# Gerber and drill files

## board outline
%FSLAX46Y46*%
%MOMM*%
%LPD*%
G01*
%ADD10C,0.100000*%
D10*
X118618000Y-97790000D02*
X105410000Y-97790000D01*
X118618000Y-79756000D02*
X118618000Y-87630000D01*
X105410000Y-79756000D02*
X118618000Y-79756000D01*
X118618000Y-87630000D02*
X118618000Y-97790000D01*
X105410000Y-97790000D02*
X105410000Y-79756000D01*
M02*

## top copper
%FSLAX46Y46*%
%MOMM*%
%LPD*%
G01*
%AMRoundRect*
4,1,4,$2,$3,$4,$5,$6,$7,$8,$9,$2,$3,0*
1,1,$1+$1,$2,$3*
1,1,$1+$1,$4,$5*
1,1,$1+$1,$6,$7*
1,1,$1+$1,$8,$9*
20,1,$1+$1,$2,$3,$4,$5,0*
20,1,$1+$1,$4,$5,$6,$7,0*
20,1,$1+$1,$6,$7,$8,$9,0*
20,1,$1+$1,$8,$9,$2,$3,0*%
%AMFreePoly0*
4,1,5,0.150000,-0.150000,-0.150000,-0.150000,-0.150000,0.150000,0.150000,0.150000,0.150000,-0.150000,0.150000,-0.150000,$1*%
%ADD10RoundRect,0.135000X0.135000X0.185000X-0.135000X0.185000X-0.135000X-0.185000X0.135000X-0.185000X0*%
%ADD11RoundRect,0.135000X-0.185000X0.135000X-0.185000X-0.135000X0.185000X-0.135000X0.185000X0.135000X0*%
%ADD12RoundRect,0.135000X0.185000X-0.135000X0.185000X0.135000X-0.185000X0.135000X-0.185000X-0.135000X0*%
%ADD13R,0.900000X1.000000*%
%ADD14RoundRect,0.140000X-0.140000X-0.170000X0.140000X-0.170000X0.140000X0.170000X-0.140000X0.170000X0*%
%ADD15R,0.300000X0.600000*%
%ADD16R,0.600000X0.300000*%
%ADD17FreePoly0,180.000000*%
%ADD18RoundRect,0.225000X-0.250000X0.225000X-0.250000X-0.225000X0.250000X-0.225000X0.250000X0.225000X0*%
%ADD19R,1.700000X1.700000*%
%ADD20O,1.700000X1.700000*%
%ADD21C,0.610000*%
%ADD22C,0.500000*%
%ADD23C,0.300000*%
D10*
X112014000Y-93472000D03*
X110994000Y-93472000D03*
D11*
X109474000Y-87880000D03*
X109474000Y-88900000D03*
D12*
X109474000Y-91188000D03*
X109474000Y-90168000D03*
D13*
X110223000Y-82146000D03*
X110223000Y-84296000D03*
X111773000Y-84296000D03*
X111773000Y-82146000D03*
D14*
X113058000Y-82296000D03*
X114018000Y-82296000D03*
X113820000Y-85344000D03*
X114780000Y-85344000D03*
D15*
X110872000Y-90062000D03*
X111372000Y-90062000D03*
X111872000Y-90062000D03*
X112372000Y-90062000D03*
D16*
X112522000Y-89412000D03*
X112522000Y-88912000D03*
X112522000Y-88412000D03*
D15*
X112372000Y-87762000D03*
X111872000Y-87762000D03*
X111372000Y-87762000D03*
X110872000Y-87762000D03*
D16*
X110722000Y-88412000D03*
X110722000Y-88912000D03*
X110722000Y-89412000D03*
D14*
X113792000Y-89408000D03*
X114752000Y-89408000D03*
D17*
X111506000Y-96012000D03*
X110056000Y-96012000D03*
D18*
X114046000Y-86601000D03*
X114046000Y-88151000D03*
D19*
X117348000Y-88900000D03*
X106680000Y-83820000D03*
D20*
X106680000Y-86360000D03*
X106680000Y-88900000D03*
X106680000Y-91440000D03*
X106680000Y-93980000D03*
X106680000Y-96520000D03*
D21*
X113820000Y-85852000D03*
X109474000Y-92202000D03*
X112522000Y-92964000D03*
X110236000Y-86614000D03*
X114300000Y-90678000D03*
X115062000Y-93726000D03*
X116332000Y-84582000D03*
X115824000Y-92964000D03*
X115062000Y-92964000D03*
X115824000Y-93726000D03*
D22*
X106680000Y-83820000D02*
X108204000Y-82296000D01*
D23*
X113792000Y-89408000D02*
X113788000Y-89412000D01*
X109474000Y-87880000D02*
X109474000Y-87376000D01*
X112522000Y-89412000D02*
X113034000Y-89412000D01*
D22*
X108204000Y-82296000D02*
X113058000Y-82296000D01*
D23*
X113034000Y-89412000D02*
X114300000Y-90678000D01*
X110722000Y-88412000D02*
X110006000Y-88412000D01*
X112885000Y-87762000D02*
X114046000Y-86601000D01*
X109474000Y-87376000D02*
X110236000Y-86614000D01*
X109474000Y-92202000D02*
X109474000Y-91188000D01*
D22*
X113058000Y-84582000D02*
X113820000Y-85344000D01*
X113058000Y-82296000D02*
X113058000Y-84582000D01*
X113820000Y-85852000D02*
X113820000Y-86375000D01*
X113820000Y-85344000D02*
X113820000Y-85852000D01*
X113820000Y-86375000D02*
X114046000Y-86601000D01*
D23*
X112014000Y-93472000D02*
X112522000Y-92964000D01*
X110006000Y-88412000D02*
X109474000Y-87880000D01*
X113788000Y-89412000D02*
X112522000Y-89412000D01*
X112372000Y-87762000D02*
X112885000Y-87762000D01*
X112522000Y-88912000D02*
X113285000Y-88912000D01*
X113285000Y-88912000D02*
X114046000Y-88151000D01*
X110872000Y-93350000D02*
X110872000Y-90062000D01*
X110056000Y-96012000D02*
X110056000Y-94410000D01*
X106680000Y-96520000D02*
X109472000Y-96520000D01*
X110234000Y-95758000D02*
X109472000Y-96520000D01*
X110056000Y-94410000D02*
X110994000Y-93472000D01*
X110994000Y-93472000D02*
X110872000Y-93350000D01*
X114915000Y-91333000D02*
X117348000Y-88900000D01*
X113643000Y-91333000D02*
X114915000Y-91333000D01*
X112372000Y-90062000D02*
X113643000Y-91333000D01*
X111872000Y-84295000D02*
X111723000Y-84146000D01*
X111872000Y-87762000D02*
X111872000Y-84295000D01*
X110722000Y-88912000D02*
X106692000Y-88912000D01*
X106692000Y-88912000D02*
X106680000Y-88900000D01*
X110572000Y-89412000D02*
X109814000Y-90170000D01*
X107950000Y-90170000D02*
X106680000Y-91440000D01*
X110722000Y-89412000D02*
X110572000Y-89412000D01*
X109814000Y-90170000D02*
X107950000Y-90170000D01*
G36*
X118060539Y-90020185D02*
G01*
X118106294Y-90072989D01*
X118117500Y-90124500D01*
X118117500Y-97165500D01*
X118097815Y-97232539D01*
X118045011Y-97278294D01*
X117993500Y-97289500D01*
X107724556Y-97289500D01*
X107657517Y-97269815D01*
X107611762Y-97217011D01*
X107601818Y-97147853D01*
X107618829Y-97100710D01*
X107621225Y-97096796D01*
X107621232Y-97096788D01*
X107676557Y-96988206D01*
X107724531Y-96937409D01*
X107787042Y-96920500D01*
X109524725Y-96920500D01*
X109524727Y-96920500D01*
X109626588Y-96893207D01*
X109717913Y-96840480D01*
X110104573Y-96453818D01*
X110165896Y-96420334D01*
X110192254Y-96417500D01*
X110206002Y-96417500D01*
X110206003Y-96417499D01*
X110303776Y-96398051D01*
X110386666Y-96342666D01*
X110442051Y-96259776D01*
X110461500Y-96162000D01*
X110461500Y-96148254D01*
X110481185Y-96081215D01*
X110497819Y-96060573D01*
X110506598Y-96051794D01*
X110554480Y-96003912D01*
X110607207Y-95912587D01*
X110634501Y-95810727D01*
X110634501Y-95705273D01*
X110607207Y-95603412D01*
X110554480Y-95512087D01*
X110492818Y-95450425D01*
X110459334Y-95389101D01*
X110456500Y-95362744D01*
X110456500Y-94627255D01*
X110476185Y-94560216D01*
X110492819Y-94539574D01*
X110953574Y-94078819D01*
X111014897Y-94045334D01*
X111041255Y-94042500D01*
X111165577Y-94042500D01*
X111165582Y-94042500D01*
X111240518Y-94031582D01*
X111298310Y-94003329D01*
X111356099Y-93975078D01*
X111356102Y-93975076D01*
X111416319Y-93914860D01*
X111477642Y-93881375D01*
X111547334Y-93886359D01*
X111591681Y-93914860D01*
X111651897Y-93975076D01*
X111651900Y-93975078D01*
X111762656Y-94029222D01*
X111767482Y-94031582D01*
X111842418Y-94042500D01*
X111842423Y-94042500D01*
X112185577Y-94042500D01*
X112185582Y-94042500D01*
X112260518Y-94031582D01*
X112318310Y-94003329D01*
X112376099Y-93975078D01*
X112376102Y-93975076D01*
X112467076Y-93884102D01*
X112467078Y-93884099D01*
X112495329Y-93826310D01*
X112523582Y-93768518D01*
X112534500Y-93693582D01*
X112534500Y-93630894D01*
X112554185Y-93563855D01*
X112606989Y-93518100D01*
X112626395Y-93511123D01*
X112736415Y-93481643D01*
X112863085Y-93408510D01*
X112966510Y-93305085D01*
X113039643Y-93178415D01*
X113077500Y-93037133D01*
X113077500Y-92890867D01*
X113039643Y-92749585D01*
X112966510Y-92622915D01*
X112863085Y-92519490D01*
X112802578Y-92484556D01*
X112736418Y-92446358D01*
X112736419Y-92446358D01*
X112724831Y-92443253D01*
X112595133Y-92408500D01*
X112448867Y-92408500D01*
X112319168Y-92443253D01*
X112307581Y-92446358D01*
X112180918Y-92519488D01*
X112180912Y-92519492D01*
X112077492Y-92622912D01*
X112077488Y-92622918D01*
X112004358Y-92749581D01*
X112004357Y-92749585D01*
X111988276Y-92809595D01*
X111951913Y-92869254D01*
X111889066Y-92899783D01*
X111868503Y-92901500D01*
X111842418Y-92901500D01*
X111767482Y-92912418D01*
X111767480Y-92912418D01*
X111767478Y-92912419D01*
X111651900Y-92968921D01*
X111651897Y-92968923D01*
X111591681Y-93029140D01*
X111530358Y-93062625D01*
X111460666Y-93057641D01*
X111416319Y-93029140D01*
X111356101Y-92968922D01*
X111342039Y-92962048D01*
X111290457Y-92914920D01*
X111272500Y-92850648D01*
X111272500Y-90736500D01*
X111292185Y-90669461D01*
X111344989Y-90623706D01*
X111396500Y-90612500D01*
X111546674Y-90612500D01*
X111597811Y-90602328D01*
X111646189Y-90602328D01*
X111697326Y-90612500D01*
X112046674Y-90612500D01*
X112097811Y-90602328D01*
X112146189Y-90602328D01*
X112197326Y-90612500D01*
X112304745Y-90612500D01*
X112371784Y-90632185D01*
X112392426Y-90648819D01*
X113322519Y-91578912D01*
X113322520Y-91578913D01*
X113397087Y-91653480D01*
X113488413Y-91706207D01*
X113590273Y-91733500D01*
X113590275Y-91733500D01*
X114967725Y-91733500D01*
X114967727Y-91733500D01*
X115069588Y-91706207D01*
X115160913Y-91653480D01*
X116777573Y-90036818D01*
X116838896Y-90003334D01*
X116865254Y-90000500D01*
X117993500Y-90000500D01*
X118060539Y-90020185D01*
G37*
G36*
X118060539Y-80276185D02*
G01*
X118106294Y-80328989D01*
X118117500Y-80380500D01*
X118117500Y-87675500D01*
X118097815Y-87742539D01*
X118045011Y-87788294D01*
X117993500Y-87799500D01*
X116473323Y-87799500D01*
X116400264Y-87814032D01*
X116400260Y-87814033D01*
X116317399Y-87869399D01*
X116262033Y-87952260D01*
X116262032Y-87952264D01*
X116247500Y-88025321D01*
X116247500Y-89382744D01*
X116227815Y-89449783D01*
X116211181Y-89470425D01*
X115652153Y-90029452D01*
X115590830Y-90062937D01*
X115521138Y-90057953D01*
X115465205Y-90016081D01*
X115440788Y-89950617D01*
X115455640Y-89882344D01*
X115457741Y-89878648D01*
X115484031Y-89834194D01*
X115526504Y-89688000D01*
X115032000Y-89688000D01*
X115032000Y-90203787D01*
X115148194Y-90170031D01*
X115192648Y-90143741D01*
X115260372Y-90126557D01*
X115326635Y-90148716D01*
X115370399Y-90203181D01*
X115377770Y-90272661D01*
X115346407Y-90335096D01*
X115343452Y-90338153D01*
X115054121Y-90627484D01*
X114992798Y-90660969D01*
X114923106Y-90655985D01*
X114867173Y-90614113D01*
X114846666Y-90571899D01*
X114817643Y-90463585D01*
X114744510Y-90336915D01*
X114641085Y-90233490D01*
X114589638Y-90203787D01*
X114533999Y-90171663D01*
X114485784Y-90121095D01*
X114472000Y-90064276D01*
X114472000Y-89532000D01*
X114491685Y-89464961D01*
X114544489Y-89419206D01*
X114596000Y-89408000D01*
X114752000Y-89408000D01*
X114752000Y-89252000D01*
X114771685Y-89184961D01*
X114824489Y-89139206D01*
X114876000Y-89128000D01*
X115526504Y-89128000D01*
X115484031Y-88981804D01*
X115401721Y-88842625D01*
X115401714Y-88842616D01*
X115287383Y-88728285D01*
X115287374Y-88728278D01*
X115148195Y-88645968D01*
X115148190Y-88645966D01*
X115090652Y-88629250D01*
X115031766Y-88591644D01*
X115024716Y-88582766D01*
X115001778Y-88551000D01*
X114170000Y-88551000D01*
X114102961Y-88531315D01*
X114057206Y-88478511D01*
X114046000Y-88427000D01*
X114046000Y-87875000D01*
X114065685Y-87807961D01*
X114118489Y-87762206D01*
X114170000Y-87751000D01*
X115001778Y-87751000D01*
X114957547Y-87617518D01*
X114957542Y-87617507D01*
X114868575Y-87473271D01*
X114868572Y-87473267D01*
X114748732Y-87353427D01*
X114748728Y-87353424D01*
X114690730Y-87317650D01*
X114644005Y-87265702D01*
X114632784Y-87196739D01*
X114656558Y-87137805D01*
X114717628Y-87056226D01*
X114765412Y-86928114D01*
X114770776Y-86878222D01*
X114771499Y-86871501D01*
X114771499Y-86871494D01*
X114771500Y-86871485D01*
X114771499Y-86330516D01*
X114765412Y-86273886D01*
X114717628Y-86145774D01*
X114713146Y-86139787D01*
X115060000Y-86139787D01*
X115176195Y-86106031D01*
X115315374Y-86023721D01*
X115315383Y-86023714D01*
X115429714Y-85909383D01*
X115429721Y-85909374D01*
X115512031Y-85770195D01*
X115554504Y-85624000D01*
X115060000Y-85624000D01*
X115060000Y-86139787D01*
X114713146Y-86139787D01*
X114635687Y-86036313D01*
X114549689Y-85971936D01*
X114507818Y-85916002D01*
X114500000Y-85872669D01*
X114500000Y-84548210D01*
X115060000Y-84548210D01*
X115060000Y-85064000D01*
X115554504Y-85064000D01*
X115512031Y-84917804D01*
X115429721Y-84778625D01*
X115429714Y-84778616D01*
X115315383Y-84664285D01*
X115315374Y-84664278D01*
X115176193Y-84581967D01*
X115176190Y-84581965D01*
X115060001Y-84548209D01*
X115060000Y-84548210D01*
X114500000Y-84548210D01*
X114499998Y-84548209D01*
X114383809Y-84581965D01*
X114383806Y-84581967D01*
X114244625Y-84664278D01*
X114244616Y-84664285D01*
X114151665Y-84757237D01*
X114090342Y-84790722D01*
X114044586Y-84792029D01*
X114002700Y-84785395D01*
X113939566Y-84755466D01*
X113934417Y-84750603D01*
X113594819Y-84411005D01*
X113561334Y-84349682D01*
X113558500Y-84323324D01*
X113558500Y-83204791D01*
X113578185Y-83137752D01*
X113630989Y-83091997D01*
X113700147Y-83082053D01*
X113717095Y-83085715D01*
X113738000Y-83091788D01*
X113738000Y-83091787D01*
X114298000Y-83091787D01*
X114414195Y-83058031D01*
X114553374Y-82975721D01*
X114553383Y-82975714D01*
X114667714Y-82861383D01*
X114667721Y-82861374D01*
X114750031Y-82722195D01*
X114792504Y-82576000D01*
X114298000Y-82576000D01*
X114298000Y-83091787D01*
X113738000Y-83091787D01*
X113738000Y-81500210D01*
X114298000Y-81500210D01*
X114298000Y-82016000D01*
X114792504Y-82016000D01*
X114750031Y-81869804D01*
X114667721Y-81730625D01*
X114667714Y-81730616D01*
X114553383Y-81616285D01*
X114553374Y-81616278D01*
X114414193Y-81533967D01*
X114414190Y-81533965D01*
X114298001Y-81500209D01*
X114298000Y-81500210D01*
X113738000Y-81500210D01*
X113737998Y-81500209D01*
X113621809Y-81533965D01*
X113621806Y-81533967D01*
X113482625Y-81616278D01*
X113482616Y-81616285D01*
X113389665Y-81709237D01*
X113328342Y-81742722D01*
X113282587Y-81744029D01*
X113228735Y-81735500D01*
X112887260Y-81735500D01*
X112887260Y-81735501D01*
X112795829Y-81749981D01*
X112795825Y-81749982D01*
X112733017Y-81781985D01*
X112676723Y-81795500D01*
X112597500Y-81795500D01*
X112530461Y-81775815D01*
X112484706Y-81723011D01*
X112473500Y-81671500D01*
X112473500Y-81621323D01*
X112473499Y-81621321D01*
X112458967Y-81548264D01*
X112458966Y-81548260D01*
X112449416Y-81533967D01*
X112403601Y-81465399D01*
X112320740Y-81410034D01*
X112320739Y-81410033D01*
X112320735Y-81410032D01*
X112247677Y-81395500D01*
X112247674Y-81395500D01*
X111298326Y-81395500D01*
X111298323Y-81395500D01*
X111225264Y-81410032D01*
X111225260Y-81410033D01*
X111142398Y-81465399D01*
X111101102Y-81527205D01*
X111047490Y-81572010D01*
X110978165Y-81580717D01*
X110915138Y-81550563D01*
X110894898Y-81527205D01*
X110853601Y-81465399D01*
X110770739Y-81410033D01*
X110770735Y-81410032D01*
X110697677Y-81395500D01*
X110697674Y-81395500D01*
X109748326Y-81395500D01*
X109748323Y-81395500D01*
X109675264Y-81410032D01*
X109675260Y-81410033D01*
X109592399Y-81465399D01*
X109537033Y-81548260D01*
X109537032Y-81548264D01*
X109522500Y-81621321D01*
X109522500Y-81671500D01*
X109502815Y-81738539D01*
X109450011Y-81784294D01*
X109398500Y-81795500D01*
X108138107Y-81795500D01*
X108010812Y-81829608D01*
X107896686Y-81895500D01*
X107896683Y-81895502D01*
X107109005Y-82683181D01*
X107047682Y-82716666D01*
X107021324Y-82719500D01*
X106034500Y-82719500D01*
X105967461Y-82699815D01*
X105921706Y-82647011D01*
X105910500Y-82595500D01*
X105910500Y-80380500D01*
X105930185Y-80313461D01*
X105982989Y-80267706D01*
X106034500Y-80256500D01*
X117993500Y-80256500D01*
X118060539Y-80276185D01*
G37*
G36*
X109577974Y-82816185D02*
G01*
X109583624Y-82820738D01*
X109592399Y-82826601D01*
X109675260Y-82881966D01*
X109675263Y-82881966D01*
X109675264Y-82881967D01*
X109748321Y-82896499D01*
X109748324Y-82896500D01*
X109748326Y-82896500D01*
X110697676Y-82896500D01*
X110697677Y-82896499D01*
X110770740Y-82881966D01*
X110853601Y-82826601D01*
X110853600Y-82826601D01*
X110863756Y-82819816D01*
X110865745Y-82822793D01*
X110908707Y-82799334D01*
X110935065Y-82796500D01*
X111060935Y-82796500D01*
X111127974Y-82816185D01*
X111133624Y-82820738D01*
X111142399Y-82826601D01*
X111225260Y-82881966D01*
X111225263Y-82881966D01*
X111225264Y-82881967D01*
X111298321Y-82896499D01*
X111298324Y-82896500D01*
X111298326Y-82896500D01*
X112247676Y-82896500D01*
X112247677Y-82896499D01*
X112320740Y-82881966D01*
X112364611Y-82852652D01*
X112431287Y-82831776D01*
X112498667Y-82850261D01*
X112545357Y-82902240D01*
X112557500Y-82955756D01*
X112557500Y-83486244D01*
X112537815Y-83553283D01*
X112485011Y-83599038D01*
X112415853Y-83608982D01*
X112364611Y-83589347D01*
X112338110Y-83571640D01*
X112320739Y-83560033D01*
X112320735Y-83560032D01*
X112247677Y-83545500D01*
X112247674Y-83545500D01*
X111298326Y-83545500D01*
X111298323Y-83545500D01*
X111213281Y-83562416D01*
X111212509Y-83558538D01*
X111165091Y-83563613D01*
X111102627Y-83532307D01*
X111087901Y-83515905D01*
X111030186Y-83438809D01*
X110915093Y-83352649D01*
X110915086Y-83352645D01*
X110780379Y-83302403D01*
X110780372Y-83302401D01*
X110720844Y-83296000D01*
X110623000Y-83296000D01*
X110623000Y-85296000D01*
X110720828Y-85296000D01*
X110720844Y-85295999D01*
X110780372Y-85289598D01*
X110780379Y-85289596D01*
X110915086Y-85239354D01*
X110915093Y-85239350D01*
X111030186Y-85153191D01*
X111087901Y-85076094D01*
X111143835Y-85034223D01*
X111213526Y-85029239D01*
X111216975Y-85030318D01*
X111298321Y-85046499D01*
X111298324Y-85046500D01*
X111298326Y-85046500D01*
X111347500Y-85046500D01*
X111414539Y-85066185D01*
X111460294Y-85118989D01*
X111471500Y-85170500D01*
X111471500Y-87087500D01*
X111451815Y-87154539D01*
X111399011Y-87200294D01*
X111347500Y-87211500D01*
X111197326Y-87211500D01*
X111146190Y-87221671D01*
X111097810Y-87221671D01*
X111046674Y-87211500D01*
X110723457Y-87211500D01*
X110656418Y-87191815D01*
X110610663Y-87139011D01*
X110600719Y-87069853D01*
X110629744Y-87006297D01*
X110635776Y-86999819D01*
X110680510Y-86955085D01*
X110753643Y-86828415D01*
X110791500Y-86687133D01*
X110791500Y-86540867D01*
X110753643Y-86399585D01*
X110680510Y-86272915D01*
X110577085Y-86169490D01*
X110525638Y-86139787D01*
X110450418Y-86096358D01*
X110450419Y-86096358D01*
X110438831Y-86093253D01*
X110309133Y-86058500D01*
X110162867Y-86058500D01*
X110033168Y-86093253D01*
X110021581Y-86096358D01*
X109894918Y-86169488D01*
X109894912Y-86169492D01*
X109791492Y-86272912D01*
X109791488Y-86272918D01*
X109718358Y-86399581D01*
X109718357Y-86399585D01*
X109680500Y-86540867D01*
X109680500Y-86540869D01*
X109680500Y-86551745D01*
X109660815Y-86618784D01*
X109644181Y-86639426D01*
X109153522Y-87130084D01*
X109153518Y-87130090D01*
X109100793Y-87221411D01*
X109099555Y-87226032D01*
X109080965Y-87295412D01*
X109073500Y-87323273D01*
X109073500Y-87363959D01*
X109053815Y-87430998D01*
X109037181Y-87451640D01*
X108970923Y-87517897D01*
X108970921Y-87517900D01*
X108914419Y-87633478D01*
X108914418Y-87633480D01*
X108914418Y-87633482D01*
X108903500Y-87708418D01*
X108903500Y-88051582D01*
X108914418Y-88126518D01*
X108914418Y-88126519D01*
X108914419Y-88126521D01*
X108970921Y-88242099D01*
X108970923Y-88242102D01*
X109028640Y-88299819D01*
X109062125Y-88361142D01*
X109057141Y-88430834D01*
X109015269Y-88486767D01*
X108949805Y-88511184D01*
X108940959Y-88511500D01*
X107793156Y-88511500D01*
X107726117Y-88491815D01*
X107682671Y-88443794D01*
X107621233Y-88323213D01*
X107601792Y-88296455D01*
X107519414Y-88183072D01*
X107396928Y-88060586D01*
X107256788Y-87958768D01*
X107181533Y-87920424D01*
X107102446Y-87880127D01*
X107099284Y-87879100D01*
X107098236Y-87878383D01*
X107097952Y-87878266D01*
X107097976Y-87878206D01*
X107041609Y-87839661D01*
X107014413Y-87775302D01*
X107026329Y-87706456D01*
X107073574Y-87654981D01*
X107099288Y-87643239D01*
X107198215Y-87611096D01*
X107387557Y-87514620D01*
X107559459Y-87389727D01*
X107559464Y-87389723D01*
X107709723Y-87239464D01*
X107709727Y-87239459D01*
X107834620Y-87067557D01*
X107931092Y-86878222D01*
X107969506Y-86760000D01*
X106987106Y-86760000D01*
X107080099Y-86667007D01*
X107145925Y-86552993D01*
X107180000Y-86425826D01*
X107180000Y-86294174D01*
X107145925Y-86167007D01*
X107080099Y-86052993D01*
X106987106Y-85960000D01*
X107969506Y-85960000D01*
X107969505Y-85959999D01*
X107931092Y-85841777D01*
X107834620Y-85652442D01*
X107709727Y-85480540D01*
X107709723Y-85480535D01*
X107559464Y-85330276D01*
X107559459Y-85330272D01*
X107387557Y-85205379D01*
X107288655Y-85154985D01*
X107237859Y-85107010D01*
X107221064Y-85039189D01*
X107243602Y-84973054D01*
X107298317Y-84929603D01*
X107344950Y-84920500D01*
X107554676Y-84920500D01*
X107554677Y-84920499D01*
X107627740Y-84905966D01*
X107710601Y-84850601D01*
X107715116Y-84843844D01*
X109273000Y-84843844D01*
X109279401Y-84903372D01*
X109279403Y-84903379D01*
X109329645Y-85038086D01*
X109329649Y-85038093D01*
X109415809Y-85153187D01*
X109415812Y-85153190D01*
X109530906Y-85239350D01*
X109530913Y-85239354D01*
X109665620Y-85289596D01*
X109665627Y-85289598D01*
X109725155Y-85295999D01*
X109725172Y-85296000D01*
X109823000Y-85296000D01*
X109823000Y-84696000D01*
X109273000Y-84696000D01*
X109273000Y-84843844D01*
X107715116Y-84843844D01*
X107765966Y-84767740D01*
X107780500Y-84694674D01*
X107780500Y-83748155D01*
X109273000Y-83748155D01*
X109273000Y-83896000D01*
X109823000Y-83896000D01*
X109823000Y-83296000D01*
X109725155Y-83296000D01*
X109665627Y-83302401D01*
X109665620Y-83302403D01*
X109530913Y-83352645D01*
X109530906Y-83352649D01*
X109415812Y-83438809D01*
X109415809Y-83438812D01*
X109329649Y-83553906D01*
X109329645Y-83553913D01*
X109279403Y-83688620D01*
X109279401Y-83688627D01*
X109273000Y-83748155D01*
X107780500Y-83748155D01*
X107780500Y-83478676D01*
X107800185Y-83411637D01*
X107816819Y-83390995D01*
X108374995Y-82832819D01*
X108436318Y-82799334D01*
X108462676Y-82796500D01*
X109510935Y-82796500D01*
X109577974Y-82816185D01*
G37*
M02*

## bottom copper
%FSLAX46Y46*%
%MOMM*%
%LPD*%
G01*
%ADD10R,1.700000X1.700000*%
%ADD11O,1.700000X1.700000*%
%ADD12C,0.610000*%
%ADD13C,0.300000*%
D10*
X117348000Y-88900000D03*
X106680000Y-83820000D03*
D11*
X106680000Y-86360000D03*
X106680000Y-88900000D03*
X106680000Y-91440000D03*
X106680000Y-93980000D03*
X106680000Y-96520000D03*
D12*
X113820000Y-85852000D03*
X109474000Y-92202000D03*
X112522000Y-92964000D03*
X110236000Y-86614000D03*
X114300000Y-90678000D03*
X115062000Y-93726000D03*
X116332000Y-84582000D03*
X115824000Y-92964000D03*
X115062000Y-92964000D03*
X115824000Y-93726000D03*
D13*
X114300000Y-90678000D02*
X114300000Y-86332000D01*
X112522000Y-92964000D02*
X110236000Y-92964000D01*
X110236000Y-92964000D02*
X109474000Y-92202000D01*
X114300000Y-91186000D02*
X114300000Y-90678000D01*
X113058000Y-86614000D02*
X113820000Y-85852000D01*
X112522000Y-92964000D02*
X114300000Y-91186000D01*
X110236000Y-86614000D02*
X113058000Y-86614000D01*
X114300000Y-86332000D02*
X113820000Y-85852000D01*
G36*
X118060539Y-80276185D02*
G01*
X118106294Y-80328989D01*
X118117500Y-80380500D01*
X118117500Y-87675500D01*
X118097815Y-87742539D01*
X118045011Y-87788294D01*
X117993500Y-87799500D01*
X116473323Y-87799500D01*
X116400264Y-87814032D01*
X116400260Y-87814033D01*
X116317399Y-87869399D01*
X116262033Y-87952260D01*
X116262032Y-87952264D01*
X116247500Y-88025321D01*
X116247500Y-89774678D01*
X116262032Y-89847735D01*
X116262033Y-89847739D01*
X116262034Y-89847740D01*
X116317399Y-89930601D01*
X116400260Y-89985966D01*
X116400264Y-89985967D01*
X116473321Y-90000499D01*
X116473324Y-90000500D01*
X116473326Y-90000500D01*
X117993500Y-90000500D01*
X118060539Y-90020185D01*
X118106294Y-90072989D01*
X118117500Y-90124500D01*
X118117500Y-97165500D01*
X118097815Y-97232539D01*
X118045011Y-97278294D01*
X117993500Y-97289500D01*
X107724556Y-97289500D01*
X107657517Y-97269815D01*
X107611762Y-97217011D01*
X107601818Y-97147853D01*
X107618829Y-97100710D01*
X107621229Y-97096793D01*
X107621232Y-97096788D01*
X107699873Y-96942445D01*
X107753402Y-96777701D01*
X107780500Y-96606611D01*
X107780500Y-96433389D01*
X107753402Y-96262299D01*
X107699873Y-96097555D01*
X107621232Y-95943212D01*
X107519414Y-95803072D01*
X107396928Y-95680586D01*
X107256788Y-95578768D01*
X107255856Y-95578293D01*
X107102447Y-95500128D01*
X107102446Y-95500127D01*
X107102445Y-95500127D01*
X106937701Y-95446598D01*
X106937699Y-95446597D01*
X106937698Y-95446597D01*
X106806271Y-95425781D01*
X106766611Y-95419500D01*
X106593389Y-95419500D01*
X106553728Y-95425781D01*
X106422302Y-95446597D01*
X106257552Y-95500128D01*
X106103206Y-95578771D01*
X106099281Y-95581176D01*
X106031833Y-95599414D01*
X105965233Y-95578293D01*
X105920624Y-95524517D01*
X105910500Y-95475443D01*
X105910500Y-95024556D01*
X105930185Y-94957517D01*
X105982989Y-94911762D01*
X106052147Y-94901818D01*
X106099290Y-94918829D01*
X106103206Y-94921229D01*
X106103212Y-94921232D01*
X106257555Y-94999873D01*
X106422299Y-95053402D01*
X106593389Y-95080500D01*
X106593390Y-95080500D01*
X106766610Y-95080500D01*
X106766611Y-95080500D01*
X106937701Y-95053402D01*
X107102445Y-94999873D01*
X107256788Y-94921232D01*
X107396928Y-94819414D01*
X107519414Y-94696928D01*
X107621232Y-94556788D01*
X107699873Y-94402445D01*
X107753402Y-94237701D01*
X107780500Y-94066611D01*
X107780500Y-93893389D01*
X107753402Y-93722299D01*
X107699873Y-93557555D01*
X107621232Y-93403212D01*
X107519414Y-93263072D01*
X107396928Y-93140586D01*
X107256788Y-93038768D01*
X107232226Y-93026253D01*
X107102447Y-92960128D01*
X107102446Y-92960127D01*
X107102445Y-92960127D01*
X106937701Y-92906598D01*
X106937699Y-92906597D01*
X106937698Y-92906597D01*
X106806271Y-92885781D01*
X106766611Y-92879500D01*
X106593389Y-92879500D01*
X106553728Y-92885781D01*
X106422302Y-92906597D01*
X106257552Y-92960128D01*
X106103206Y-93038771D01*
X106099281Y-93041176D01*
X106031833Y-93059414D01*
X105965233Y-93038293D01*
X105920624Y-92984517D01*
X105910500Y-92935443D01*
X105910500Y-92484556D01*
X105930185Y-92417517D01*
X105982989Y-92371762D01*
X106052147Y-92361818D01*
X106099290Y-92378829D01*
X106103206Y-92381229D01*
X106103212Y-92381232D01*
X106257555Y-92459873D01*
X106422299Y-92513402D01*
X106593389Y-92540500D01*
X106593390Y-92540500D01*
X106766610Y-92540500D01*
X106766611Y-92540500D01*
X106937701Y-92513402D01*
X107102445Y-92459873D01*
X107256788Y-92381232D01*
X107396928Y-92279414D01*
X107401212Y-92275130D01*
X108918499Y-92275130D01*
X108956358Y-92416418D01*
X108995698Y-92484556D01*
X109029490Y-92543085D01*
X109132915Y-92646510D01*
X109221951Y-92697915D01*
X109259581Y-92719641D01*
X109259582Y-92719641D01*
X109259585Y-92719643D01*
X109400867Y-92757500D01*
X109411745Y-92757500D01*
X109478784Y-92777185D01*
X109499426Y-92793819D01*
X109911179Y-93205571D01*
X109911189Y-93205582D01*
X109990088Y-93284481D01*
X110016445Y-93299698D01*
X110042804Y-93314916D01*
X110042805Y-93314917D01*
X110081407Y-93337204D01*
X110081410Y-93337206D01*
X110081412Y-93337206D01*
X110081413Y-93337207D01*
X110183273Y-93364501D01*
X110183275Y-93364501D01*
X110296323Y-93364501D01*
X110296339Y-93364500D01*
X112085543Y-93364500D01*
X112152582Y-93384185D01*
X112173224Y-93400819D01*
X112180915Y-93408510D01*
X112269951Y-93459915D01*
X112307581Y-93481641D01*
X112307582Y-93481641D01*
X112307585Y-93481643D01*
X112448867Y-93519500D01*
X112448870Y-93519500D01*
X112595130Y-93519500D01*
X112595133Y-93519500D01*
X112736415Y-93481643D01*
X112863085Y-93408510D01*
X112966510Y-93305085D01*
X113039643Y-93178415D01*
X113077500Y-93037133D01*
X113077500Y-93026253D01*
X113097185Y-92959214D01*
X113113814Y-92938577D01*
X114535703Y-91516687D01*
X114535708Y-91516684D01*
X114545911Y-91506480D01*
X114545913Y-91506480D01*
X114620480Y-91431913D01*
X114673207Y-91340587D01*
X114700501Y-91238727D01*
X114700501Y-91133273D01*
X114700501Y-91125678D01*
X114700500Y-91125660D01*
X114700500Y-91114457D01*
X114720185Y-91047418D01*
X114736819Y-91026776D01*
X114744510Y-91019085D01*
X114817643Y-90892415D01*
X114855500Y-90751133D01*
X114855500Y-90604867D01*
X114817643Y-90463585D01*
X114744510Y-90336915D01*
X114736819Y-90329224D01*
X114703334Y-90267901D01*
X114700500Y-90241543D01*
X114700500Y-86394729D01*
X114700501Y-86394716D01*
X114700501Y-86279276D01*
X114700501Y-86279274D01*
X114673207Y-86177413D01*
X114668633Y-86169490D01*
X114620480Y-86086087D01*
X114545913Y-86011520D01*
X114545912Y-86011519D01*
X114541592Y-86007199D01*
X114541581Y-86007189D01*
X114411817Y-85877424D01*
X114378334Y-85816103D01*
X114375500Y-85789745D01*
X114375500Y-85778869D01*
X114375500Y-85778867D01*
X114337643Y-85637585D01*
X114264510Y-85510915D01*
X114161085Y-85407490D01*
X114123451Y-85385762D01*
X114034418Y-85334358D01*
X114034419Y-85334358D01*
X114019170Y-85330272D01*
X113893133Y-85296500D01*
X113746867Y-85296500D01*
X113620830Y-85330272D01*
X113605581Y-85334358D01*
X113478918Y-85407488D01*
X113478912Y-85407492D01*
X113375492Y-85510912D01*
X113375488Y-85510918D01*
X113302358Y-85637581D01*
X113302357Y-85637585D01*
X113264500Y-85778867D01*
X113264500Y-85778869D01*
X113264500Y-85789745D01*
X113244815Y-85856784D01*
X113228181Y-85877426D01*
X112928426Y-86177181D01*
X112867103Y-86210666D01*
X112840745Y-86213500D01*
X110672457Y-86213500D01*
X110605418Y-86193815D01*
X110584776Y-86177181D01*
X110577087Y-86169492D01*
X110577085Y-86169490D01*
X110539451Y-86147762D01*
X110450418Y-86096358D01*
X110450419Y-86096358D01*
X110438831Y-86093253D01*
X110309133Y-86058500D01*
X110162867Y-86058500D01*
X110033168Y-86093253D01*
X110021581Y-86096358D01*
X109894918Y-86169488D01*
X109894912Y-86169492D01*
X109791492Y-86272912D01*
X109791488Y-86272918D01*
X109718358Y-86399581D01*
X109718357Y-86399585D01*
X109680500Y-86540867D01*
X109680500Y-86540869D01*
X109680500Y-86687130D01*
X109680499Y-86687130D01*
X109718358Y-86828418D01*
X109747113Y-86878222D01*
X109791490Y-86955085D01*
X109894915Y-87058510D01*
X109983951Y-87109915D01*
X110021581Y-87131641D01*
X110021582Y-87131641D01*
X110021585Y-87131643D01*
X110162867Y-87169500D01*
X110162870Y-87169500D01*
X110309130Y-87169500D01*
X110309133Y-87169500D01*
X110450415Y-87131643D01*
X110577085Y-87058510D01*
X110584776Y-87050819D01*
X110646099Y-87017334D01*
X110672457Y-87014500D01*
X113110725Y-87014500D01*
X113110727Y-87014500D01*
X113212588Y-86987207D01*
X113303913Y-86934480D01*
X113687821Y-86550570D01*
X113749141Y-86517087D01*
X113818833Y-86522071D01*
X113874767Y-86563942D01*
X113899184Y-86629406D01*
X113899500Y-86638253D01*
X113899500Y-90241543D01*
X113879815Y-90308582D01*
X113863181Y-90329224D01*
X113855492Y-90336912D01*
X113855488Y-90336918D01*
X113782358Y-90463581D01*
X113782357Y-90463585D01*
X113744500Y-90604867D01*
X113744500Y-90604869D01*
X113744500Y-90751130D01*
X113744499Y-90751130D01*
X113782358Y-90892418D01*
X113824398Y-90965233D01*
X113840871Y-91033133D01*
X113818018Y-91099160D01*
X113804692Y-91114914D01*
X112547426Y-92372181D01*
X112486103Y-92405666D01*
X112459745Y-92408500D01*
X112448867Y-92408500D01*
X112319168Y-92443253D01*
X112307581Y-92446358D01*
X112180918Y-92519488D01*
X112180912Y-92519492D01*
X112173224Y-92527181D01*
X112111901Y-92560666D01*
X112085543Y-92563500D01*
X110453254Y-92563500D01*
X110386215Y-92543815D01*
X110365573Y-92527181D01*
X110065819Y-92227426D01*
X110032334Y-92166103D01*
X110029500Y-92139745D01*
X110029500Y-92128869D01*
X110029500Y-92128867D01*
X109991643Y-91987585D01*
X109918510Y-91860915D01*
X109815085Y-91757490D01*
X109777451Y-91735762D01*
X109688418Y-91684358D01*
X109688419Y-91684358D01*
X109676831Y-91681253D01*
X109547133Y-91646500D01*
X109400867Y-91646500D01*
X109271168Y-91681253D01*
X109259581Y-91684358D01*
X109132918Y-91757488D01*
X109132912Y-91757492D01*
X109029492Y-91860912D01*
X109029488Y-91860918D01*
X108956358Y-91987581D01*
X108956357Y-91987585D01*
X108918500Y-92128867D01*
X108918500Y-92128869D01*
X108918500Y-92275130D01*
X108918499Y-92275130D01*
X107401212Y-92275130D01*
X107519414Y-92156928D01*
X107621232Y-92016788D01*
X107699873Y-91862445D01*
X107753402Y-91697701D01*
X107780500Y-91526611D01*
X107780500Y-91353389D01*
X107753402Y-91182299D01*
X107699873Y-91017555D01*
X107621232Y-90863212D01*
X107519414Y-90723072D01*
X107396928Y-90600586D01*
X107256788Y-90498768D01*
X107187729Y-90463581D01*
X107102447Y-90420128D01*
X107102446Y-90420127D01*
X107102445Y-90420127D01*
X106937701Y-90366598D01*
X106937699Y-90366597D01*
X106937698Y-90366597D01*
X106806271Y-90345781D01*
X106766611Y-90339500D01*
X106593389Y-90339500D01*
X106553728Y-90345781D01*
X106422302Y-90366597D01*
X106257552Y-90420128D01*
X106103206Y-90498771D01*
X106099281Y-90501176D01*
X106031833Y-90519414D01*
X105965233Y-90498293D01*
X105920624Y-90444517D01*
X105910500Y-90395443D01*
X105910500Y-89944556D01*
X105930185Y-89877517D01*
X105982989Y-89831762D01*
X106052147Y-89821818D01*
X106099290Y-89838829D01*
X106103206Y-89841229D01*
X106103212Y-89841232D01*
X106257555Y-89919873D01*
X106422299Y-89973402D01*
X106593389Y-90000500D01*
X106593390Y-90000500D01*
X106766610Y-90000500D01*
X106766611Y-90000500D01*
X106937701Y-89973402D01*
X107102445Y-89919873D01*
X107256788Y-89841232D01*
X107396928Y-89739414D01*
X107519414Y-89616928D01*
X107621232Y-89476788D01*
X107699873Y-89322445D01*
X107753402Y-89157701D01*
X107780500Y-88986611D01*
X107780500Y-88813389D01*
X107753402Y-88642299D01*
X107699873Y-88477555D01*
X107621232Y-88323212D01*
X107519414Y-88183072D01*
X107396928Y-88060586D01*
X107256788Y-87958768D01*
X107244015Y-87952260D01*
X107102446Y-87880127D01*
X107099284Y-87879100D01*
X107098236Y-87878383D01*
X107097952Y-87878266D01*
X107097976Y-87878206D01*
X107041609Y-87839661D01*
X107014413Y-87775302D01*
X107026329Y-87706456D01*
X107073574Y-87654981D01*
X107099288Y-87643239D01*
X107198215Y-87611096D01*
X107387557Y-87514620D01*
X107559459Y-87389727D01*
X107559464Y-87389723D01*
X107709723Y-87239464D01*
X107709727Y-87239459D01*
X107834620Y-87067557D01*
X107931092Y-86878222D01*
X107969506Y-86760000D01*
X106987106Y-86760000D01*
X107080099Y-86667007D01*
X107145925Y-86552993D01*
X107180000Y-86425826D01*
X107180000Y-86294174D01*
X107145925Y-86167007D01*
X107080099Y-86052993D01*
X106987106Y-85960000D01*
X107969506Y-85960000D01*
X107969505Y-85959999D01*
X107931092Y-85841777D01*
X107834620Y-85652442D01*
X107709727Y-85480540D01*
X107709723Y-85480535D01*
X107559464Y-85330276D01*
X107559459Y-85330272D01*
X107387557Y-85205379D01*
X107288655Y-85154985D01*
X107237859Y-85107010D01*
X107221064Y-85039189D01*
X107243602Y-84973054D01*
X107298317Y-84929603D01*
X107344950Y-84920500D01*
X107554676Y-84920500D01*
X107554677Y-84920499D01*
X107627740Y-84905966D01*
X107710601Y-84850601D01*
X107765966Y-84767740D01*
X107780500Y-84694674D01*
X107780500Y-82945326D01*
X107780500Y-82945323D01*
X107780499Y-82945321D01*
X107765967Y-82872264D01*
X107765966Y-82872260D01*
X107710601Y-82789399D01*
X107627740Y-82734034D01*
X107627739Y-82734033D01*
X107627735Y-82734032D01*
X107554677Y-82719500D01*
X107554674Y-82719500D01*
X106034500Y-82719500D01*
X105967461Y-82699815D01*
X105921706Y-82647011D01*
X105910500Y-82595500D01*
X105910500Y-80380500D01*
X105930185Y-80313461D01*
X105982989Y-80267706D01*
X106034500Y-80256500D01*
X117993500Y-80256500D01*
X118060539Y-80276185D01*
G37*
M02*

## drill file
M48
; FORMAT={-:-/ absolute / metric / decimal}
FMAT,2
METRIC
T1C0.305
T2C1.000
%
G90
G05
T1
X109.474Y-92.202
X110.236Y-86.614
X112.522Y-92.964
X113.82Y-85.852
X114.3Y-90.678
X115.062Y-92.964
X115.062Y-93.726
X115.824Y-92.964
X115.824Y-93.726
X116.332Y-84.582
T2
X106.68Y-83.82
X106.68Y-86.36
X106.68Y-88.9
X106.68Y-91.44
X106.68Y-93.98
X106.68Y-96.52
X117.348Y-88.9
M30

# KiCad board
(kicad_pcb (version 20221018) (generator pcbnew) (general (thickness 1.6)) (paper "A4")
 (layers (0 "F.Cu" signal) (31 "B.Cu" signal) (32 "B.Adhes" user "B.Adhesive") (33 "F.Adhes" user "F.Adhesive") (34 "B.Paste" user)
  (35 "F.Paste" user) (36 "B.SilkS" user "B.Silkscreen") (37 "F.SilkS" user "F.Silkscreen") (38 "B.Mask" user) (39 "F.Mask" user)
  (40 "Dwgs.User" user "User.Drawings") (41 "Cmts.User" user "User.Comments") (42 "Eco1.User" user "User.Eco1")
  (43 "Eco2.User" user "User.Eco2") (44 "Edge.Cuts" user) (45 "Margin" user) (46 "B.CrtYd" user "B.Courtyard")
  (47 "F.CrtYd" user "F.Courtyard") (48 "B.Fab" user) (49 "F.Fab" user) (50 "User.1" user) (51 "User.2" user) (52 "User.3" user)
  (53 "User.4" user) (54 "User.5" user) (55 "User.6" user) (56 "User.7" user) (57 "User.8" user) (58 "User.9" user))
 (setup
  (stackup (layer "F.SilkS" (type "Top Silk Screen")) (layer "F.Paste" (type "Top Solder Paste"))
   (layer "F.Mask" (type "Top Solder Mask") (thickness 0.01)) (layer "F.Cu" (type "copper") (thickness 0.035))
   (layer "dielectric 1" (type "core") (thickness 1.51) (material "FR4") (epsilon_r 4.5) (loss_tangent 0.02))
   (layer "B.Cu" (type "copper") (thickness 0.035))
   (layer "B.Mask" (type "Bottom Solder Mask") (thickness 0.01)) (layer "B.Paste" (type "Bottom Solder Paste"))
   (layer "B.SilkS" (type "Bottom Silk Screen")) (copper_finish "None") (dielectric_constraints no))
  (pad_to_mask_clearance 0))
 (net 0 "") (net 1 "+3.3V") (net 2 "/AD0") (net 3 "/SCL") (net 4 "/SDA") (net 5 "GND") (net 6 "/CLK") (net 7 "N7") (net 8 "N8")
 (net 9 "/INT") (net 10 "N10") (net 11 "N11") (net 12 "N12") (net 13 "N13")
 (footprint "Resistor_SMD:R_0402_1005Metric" (layer "F.Cu") (at 111.504 93.472 180)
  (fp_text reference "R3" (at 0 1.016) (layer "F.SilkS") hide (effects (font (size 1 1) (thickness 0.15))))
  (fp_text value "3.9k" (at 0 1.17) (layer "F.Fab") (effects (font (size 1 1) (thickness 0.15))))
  (pad "1" smd roundrect (at -0.51 0 180) (size 0.54 0.64) (layers "F.Cu" "F.Paste" "F.Mask") (roundrect_rratio 0.25) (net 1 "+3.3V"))
  (pad "2" smd roundrect (at 0.51 0 180) (size 0.54 0.64) (layers "F.Cu" "F.Paste" "F.Mask") (roundrect_rratio 0.25) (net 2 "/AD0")))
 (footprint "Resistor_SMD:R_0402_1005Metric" (layer "F.Cu") (at 109.474 88.39 -90)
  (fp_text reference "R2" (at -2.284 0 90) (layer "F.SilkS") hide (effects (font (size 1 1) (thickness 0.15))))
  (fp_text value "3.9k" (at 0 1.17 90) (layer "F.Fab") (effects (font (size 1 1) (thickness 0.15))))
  (pad "1" smd roundrect (at -0.51 0 270) (size 0.54 0.64) (layers "F.Cu" "F.Paste" "F.Mask") (roundrect_rratio 0.25) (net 1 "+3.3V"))
  (pad "2" smd roundrect (at 0.51 0 270) (size 0.54 0.64) (layers "F.Cu" "F.Paste" "F.Mask") (roundrect_rratio 0.25) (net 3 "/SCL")))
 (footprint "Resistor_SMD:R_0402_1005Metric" (layer "F.Cu") (at 109.474 90.678 90)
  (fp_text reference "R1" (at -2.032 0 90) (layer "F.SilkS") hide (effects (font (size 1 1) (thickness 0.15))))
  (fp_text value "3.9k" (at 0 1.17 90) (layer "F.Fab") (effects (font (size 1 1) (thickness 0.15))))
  (pad "1" smd roundrect (at -0.51 0 90) (size 0.54 0.64) (layers "F.Cu" "F.Paste" "F.Mask") (roundrect_rratio 0.25) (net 1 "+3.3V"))
  (pad "2" smd roundrect (at 0.51 0 90) (size 0.54 0.64) (layers "F.Cu" "F.Paste" "F.Mask") (roundrect_rratio 0.25) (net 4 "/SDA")))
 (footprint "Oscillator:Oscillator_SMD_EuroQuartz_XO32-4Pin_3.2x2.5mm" (layer "F.Cu") (at 110.998 83.221)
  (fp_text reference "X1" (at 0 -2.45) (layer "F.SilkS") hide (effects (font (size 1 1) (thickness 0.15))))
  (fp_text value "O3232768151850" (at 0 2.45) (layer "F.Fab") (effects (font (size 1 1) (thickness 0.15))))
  (pad "1" smd rect (at -0.775 -1.075 270) (size 1 0.9) (layers "F.Cu" "F.Paste" "F.Mask") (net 1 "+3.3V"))
  (pad "2" smd rect (at -0.775 1.075 270) (size 1 0.9) (layers "F.Cu" "F.Paste" "F.Mask") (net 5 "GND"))
  (pad "3" smd rect (at 0.775 1.075 270) (size 1 0.9) (layers "F.Cu" "F.Paste" "F.Mask") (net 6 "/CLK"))
  (pad "4" smd rect (at 0.775 -1.075 270) (size 1 0.9) (layers "F.Cu" "F.Paste" "F.Mask") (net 1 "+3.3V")))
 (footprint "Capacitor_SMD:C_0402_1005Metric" (layer "F.Cu") (at 113.538 82.296)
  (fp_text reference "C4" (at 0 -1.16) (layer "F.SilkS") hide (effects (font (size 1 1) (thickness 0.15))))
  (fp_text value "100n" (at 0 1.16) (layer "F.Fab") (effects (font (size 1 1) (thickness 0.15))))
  (pad "1" smd roundrect (at -0.48 0) (size 0.56 0.62) (layers "F.Cu" "F.Paste" "F.Mask") (roundrect_rratio 0.25) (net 1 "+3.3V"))
  (pad "2" smd roundrect (at 0.48 0) (size 0.56 0.62) (layers "F.Cu" "F.Paste" "F.Mask") (roundrect_rratio 0.25) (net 5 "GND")))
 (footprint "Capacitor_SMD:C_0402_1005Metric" (layer "F.Cu") (at 114.3 85.344)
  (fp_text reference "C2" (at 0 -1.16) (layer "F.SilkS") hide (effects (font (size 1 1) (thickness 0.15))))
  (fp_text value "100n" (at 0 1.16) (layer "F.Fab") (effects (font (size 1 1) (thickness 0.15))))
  (pad "1" smd roundrect (at -0.48 0) (size 0.56 0.62) (layers "F.Cu" "F.Paste" "F.Mask") (roundrect_rratio 0.25) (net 1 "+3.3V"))
  (pad "2" smd roundrect (at 0.48 0) (size 0.56 0.62) (layers "F.Cu" "F.Paste" "F.Mask") (roundrect_rratio 0.25) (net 5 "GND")))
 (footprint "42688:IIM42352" (layer "F.Cu") (at 111.622 88.912 90)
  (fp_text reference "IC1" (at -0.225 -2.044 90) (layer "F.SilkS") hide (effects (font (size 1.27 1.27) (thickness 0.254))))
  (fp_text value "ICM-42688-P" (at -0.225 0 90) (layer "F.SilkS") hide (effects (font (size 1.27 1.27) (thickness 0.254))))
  (pad "1" smd rect (at -1.15 -0.75 180) (size 0.3 0.6) (layers "F.Cu" "F.Paste" "F.Mask") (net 2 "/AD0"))
  (pad "2" smd rect (at -1.15 -0.25 180) (size 0.3 0.6) (layers "F.Cu" "F.Paste" "F.Mask") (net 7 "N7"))
  (pad "3" smd rect (at -1.15 0.25 180) (size 0.3 0.6) (layers "F.Cu" "F.Paste" "F.Mask") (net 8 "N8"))
  (pad "4" smd rect (at -1.15 0.75 180) (size 0.3 0.6) (layers "F.Cu" "F.Paste" "F.Mask") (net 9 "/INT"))
  (pad "5" smd rect (at -0.5 0.9 90) (size 0.3 0.6) (layers "F.Cu" "F.Paste" "F.Mask") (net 1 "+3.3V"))
  (pad "6" smd rect (at 0 0.9 90) (size 0.3 0.6) (layers "F.Cu" "F.Paste" "F.Mask") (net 5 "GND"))
  (pad "7" smd rect (at 0.5 0.9 90) (size 0.3 0.6) (layers "F.Cu" "F.Paste" "F.Mask") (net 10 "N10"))
  (pad "8" smd rect (at 1.15 0.75 180) (size 0.3 0.6) (layers "F.Cu" "F.Paste" "F.Mask") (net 1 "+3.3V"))
  (pad "9" smd rect (at 1.15 0.25 180) (size 0.3 0.6) (layers "F.Cu" "F.Paste" "F.Mask") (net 6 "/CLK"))
  (pad "10" smd rect (at 1.15 -0.25 180) (size 0.3 0.6) (layers "F.Cu" "F.Paste" "F.Mask") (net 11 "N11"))
  (pad "11" smd rect (at 1.15 -0.75 180) (size 0.3 0.6) (layers "F.Cu" "F.Paste" "F.Mask") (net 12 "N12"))
  (pad "12" smd rect (at 0.5 -0.9 90) (size 0.3 0.6) (layers "F.Cu" "F.Paste" "F.Mask") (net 1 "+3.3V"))
  (pad "13" smd rect (at 0 -0.9 90) (size 0.3 0.6) (layers "F.Cu" "F.Paste" "F.Mask") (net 3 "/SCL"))
  (pad "14" smd rect (at -0.5 -0.9 90) (size 0.3 0.6) (layers "F.Cu" "F.Paste" "F.Mask") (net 4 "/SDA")))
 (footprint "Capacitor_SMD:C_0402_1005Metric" (layer "F.Cu") (at 114.272 89.408)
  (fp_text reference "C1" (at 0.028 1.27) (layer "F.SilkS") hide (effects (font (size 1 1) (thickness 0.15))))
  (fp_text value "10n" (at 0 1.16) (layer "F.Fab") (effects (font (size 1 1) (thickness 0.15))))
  (pad "1" smd roundrect (at -0.48 0) (size 0.56 0.62) (layers "F.Cu" "F.Paste" "F.Mask") (roundrect_rratio 0.25) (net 1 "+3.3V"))
  (pad "2" smd roundrect (at 0.48 0) (size 0.56 0.62) (layers "F.Cu" "F.Paste" "F.Mask") (roundrect_rratio 0.25) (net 5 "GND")))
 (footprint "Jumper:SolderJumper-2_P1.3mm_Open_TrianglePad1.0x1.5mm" (layer "F.Cu") (at 110.781 96.012 180)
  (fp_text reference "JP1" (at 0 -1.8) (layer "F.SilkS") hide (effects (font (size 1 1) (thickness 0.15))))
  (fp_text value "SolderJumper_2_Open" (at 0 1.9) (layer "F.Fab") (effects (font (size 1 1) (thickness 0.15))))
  (pad "1" smd custom (at -0.725 0 180) (size 0.3 0.3) (layers "F.Cu" "F.Mask") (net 5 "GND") (zone_connect 2) (thermal_bridge_angle 45)
   (options (clearance outline) (anchor rect)) (primitives))
  (pad "2" smd custom (at 0.725 0 180) (size 0.3 0.3) (layers "F.Cu" "F.Mask") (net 2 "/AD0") (zone_connect 2) (thermal_bridge_angle 45)
   (options (clearance outline) (anchor rect)) (primitives)))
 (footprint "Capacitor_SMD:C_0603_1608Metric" (layer "F.Cu") (at 114.046 87.376 -90)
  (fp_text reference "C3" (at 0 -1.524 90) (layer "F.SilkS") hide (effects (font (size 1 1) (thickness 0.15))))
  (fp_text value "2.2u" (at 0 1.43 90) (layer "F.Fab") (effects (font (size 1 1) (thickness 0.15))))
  (pad "1" smd roundrect (at -0.775 0 270) (size 0.9 0.95) (layers "F.Cu" "F.Paste" "F.Mask") (roundrect_rratio 0.25) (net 1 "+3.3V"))
  (pad "2" smd roundrect (at 0.775 0 270) (size 0.9 0.95) (layers "F.Cu" "F.Paste" "F.Mask") (roundrect_rratio 0.25) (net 5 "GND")))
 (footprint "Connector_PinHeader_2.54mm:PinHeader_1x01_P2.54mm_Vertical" (layer "B.Cu") (at 117.348 88.9 180)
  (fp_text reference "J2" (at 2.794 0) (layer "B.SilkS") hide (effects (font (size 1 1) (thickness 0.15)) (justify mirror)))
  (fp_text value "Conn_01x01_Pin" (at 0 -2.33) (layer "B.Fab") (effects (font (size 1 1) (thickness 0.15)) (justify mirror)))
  (pad "1" thru_hole rect (at 0 0 180) (size 1.7 1.7) (drill 1) (layers "*.Cu" "*.Mask") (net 9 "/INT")))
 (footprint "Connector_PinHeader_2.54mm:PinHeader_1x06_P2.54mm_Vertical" (layer "B.Cu") (at 106.68 83.82 180)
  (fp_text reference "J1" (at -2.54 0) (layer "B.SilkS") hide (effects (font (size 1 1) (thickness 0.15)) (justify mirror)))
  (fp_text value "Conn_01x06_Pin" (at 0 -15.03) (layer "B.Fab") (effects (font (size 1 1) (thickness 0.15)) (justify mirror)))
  (pad "1" thru_hole rect (at 0 0 180) (size 1.7 1.7) (drill 1) (layers "*.Cu" "*.Mask") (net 1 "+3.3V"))
  (pad "2" thru_hole oval (at 0 -2.54 180) (size 1.7 1.7) (drill 1) (layers "*.Cu" "*.Mask") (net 5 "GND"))
  (pad "3" thru_hole oval (at 0 -5.08 180) (size 1.7 1.7) (drill 1) (layers "*.Cu" "*.Mask") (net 3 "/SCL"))
  (pad "4" thru_hole oval (at 0 -7.62 180) (size 1.7 1.7) (drill 1) (layers "*.Cu" "*.Mask") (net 4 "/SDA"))
  (pad "5" thru_hole oval (at 0 -10.16 180) (size 1.7 1.7) (drill 1) (layers "*.Cu" "*.Mask") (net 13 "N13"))
  (pad "6" thru_hole oval (at 0 -12.7 180) (size 1.7 1.7) (drill 1) (layers "*.Cu" "*.Mask") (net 2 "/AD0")))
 (gr_line (start 118.618 97.79) (end 105.41 97.79) (stroke (width 0.1) (type default)) (layer "Edge.Cuts"))
 (gr_line (start 118.618 79.756) (end 118.618 87.63) (stroke (width 0.1) (type default)) (layer "Edge.Cuts"))
 (gr_line (start 105.41 79.756) (end 118.618 79.756) (stroke (width 0.1) (type default)) (layer "Edge.Cuts"))
 (gr_line (start 118.618 87.63) (end 118.618 97.79) (stroke (width 0.1) (type default)) (layer "Edge.Cuts"))
 (gr_line (start 105.41 97.79) (end 105.41 79.756) (stroke (width 0.1) (type default)) (layer "Edge.Cuts"))
 (segment (start 106.68 83.82) (end 108.204 82.296) (width 0.5) (layer "F.Cu") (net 1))
 (segment (start 113.792 89.408) (end 113.788 89.412) (width 0.3) (layer "F.Cu") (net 1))
 (segment (start 109.474 87.88) (end 109.474 87.376) (width 0.3) (layer "F.Cu") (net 1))
 (segment (start 112.522 89.412) (end 113.034 89.412) (width 0.3) (layer "F.Cu") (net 1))
 (segment (start 108.204 82.296) (end 113.058 82.296) (width 0.5) (layer "F.Cu") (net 1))
 (segment (start 113.034 89.412) (end 114.3 90.678) (width 0.3) (layer "F.Cu") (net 1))
 (segment (start 110.722 88.412) (end 110.006 88.412) (width 0.3) (layer "F.Cu") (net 1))
 (segment (start 112.885 87.762) (end 114.046 86.601) (width 0.3) (layer "F.Cu") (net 1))
 (segment (start 109.474 87.376) (end 110.236 86.614) (width 0.3) (layer "F.Cu") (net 1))
 (segment (start 109.474 92.202) (end 109.474 91.188) (width 0.3) (layer "F.Cu") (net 1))
 (segment (start 113.058 84.582) (end 113.82 85.344) (width 0.5) (layer "F.Cu") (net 1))
 (segment (start 113.058 82.296) (end 113.058 84.582) (width 0.5) (layer "F.Cu") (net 1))
 (segment (start 113.82 85.852) (end 113.82 86.375) (width 0.5) (layer "F.Cu") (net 1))
 (segment (start 113.82 85.344) (end 113.82 85.852) (width 0.5) (layer "F.Cu") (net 1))
 (segment (start 113.82 86.375) (end 114.046 86.601) (width 0.5) (layer "F.Cu") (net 1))
 (segment (start 112.014 93.472) (end 112.522 92.964) (width 0.3) (layer "F.Cu") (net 1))
 (segment (start 110.006 88.412) (end 109.474 87.88) (width 0.3) (layer "F.Cu") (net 1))
 (segment (start 113.788 89.412) (end 112.522 89.412) (width 0.3) (layer "F.Cu") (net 1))
 (segment (start 112.372 87.762) (end 112.885 87.762) (width 0.3) (layer "F.Cu") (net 1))
 (via (at 113.82 85.852) (size 0.61) (drill 0.305) (layers "F.Cu" "B.Cu") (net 1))
 (via (at 109.474 92.202) (size 0.61) (drill 0.305) (layers "F.Cu" "B.Cu") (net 1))
 (via (at 112.522 92.964) (size 0.61) (drill 0.305) (layers "F.Cu" "B.Cu") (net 1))
 (via (at 110.236 86.614) (size 0.61) (drill 0.305) (layers "F.Cu" "B.Cu") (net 1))
 (via (at 114.3 90.678) (size 0.61) (drill 0.305) (layers "F.Cu" "B.Cu") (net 1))
 (segment (start 114.3 90.678) (end 114.3 86.332) (width 0.3) (layer "B.Cu") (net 1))
 (segment (start 112.522 92.964) (end 110.236 92.964) (width 0.3) (layer "B.Cu") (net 1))
 (segment (start 110.236 92.964) (end 109.474 92.202) (width 0.3) (layer "B.Cu") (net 1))
 (segment (start 114.3 91.186) (end 114.3 90.678) (width 0.3) (layer "B.Cu") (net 1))
 (segment (start 113.058 86.614) (end 113.82 85.852) (width 0.3) (layer "B.Cu") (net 1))
 (segment (start 112.522 92.964) (end 114.3 91.186) (width 0.3) (layer "B.Cu") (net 1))
 (segment (start 110.236 86.614) (end 113.058 86.614) (width 0.3) (layer "B.Cu") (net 1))
 (segment (start 114.3 86.332) (end 113.82 85.852) (width 0.3) (layer "B.Cu") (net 1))
 (segment (start 112.522 88.912) (end 113.285 88.912) (width 0.3) (layer "F.Cu") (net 5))
 (segment (start 113.285 88.912) (end 114.046 88.151) (width 0.3) (layer "F.Cu") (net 5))
 (via (at 115.062 93.726) (size 0.61) (drill 0.305) (layers "F.Cu" "B.Cu") (free) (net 5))
 (via (at 116.332 84.582) (size 0.61) (drill 0.305) (layers "F.Cu" "B.Cu") (free) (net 5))
 (via (at 115.824 92.964) (size 0.61) (drill 0.305) (layers "F.Cu" "B.Cu") (free) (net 5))
 (via (at 115.062 92.964) (size 0.61) (drill 0.305) (layers "F.Cu" "B.Cu") (free) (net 5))
 (via (at 115.824 93.726) (size 0.61) (drill 0.305) (layers "F.Cu" "B.Cu") (free) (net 5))
 (segment (start 110.872 93.35) (end 110.872 90.062) (width 0.3) (layer "F.Cu") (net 2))
 (segment (start 110.056 96.012) (end 110.056 94.41) (width 0.3) (layer "F.Cu") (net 2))
 (segment (start 106.68 96.52) (end 109.472 96.52) (width 0.3) (layer "F.Cu") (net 2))
 (segment (start 110.234 95.758) (end 109.472 96.52) (width 0.3) (layer "F.Cu") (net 2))
 (segment (start 110.056 94.41) (end 110.994 93.472) (width 0.3) (layer "F.Cu") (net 2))
 (segment (start 110.994 93.472) (end 110.872 93.35) (width 0.3) (layer "F.Cu") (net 2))
 (segment (start 114.915 91.333) (end 117.348 88.9) (width 0.3) (layer "F.Cu") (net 9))
 (segment (start 113.643 91.333) (end 114.915 91.333) (width 0.3) (layer "F.Cu") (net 9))
 (segment (start 112.372 90.062) (end 113.643 91.333) (width 0.3) (layer "F.Cu") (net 9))
 (segment (start 111.872 84.295) (end 111.723 84.146) (width 0.3) (layer "F.Cu") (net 6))
 (segment (start 111.872 87.762) (end 111.872 84.295) (width 0.3) (layer "F.Cu") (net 6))
 (segment (start 110.722 88.912) (end 106.692 88.912) (width 0.3) (layer "F.Cu") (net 3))
 (segment (start 106.692 88.912) (end 106.68 88.9) (width 0.3) (layer "F.Cu") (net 3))
 (segment (start 110.572 89.412) (end 109.814 90.17) (width 0.3) (layer "F.Cu") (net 4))
 (segment (start 107.95 90.17) (end 106.68 91.44) (width 0.3) (layer "F.Cu") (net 4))
 (segment (start 110.722 89.412) (end 110.572 89.412) (width 0.3) (layer "F.Cu") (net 4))
 (segment (start 109.814 90.17) (end 107.95 90.17) (width 0.3) (layer "F.Cu") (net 4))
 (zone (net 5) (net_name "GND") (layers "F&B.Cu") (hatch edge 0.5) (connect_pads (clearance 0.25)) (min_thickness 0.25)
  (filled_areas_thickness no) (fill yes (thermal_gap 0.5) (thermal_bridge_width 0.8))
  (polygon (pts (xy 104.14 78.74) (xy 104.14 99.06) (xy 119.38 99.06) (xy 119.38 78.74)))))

